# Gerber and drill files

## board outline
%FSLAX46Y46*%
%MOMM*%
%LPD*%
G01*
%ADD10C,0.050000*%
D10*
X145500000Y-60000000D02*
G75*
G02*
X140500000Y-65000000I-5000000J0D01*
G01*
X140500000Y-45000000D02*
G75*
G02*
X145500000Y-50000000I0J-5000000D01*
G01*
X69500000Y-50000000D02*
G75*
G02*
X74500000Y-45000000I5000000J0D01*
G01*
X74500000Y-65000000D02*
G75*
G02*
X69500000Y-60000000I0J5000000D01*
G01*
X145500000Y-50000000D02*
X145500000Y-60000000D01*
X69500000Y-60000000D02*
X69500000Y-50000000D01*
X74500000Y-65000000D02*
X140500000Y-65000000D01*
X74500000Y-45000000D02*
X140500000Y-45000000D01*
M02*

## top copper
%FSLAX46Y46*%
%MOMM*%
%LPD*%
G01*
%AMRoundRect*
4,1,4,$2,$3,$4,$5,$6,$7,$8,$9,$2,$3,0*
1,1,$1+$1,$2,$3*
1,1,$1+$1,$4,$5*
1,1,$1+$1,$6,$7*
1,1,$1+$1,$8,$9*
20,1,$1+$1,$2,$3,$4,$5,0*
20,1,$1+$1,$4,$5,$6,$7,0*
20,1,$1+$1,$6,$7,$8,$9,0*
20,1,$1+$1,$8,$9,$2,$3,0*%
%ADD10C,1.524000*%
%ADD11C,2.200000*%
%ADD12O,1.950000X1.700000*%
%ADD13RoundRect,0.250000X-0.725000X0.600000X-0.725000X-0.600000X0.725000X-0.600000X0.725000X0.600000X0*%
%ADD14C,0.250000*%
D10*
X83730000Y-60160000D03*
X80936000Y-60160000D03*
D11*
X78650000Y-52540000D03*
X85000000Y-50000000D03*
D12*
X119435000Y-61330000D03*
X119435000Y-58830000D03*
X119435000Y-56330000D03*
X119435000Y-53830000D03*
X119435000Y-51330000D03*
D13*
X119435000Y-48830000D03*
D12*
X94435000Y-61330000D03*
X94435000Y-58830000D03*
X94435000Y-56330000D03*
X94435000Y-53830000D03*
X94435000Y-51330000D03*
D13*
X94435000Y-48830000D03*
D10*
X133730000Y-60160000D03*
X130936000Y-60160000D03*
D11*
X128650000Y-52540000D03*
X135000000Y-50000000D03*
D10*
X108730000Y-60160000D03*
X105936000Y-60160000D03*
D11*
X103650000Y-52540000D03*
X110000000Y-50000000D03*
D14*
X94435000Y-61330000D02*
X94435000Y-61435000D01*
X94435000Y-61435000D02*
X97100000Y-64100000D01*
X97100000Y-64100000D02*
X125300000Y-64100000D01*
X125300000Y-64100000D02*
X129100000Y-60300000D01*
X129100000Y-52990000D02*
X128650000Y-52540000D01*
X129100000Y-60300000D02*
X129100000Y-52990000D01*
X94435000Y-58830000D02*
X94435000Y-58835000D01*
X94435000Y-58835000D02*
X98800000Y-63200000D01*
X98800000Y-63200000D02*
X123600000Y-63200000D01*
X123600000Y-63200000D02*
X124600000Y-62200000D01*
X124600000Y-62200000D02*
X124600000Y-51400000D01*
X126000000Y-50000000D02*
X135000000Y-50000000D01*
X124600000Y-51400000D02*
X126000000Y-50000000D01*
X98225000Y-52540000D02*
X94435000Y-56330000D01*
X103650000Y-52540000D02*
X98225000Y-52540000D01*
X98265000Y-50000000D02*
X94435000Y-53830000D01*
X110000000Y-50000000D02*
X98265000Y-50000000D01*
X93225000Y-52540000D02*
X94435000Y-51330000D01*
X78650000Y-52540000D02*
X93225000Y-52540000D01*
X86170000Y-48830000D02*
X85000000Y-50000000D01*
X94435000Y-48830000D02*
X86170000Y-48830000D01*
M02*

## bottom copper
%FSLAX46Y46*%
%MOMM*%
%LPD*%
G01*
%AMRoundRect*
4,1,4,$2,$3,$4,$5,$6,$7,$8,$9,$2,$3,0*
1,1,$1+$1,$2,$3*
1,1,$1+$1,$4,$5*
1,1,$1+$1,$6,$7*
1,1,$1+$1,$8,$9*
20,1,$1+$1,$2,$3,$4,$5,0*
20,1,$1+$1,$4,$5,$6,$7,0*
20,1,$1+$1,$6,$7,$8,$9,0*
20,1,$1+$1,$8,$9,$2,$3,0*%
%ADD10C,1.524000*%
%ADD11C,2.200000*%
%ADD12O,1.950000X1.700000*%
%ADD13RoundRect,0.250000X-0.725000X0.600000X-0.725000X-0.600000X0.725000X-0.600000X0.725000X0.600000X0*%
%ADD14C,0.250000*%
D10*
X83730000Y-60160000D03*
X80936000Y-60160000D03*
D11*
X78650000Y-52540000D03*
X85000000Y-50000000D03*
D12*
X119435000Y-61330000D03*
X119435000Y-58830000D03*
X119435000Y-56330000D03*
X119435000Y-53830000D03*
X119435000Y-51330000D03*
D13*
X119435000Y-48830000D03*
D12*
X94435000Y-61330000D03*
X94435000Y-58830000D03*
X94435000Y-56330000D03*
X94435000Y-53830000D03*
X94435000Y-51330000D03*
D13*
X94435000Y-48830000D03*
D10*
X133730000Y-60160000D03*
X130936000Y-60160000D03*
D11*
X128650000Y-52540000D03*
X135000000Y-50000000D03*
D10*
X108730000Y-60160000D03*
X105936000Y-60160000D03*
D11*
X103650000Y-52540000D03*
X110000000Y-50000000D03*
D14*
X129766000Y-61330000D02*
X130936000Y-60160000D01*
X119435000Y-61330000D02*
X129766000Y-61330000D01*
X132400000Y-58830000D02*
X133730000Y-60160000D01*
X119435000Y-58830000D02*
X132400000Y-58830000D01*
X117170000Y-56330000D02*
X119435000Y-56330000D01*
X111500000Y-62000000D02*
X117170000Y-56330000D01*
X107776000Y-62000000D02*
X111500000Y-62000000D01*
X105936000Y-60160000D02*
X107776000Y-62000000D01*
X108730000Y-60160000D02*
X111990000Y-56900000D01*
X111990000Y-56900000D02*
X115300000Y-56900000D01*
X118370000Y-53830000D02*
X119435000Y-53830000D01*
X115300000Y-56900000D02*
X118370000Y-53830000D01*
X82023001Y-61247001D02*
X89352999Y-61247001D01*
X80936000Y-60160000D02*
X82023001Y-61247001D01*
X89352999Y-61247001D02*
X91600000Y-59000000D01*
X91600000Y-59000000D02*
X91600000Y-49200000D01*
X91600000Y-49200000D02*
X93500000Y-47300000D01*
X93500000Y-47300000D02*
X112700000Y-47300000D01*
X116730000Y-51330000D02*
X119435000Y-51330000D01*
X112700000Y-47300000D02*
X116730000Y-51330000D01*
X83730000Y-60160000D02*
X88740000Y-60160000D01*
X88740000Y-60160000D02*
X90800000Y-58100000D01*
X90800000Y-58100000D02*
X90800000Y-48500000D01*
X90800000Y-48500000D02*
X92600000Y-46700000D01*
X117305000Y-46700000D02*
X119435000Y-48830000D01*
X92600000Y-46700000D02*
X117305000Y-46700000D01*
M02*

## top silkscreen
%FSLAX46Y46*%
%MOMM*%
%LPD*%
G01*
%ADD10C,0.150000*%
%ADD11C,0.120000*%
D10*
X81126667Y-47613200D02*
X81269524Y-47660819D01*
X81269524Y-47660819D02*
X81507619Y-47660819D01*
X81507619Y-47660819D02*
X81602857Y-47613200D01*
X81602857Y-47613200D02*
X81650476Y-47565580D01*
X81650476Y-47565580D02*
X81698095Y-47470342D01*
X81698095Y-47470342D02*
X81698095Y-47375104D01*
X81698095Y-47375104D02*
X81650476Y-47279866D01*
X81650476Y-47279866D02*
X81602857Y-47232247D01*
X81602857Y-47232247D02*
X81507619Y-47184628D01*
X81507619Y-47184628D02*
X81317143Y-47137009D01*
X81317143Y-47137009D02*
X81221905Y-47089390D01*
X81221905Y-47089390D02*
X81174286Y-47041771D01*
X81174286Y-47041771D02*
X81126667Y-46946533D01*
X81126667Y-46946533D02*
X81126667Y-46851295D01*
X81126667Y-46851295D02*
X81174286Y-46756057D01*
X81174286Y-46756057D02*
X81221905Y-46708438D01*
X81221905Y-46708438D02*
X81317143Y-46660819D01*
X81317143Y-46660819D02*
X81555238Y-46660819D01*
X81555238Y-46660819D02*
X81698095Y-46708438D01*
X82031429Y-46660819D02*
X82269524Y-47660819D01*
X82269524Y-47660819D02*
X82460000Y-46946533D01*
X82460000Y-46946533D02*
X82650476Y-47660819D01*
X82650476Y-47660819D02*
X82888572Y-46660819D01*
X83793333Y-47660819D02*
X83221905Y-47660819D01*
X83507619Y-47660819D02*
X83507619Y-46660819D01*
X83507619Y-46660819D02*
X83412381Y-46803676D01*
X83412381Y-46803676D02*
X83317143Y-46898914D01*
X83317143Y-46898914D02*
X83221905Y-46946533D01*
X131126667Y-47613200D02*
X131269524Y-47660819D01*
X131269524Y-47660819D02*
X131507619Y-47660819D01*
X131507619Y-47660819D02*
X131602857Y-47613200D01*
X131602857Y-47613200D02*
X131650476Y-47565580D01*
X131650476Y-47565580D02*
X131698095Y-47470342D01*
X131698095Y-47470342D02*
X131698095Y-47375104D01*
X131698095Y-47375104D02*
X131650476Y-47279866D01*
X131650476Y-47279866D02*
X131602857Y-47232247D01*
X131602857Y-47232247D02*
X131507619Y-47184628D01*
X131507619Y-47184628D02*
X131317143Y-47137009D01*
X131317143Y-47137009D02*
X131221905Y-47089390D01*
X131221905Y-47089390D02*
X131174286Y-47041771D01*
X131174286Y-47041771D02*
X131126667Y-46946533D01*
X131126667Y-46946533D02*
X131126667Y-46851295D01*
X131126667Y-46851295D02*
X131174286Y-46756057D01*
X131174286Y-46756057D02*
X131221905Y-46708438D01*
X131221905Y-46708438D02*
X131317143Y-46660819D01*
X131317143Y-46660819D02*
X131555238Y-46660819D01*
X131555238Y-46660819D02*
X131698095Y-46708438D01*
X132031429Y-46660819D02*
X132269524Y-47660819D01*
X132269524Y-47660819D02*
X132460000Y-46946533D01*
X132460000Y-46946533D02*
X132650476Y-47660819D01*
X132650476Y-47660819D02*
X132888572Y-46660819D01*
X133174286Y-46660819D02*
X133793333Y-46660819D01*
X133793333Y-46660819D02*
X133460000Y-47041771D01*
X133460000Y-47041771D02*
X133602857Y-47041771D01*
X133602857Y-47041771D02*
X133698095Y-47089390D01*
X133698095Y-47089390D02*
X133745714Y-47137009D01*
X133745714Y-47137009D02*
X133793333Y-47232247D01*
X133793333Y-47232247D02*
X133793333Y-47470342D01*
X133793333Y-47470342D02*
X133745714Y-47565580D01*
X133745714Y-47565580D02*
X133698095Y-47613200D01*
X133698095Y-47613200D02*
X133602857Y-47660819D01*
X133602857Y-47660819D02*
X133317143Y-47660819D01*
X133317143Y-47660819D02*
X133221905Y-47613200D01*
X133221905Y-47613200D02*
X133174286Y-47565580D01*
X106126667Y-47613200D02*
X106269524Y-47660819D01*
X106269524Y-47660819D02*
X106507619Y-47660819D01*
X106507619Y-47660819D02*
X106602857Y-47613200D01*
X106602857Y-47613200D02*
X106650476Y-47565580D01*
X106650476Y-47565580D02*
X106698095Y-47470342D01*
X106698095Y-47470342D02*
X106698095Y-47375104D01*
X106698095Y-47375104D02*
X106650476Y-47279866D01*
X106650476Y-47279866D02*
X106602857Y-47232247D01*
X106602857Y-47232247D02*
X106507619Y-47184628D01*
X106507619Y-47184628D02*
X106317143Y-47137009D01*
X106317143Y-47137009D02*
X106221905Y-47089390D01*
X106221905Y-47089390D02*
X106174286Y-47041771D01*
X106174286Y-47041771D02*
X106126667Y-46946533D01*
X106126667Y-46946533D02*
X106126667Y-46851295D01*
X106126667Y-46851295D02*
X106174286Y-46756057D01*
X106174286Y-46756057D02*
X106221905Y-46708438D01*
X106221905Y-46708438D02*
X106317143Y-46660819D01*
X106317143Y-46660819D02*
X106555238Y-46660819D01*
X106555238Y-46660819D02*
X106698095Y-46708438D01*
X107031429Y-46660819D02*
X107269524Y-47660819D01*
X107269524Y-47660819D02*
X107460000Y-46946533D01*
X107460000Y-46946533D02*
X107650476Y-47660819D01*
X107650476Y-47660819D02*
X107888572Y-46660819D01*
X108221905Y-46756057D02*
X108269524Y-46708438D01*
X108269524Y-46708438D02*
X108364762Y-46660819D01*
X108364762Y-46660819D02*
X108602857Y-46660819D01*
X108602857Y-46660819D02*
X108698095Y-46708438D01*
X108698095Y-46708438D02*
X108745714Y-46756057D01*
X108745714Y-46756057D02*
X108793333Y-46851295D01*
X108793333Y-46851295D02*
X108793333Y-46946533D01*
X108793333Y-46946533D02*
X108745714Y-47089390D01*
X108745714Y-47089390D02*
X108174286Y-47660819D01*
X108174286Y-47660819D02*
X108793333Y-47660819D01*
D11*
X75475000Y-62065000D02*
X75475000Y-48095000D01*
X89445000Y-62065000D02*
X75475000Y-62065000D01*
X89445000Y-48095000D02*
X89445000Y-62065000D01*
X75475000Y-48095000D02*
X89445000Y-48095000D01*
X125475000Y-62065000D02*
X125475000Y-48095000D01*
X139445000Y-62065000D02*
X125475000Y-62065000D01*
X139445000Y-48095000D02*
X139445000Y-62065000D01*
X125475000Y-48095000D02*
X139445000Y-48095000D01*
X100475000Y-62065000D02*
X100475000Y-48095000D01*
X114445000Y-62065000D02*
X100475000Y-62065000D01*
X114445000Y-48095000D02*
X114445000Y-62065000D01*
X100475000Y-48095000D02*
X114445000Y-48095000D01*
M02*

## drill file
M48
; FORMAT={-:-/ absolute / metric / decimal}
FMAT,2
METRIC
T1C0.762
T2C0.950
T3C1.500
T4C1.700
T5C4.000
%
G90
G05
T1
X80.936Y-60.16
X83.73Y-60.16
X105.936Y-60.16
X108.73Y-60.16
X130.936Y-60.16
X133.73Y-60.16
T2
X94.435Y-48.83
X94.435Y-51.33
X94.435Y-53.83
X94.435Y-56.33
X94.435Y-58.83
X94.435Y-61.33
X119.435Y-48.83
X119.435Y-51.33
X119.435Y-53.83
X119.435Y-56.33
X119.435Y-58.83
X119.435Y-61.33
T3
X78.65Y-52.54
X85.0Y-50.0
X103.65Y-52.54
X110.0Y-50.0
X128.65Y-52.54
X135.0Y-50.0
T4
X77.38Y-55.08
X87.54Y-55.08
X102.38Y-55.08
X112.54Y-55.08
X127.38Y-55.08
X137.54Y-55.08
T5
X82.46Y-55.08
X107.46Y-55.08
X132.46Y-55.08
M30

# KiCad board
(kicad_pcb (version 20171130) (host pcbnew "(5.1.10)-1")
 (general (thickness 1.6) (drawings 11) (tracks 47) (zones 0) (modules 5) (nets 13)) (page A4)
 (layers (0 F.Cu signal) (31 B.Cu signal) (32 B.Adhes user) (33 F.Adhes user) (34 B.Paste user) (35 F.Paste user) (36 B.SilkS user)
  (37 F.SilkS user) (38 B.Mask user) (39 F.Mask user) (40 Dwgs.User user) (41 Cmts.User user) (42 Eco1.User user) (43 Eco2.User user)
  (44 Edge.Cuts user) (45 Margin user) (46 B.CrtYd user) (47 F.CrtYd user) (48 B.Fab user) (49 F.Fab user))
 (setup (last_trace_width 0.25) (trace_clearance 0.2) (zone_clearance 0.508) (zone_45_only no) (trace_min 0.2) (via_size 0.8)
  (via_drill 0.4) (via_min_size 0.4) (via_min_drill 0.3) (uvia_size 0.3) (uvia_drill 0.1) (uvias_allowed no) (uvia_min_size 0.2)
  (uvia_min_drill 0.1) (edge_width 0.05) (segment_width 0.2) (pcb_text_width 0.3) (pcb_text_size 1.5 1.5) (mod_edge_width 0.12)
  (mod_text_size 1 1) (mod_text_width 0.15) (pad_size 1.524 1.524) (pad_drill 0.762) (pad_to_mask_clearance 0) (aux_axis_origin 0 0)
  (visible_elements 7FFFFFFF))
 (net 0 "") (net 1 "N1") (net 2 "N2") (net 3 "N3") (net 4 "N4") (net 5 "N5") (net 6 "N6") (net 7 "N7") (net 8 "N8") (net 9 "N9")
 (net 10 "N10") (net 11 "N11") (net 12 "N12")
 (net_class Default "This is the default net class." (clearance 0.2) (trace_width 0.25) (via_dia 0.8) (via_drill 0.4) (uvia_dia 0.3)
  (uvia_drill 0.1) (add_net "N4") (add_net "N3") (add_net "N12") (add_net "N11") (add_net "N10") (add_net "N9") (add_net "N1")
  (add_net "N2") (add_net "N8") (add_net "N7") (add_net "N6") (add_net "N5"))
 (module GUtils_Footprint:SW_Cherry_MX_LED (layer F.Cu) (at 85 50)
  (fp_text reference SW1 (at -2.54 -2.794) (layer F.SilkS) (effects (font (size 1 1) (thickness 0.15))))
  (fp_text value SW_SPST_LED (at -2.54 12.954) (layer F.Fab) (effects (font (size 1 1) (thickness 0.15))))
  (fp_line (start -9.525 12.065) (end -9.525 -1.905) (layer F.SilkS) (width 0.12))
  (fp_line (start 4.445 12.065) (end -9.525 12.065) (layer F.SilkS) (width 0.12))
  (fp_line (start 4.445 -1.905) (end 4.445 12.065) (layer F.SilkS) (width 0.12))
  (fp_line (start -9.525 -1.905) (end 4.445 -1.905) (layer F.SilkS) (width 0.12))
  (pad 4 thru_hole circle (at -1.27 10.16) (size 1.524 1.524) (drill 0.762) (layers *.Cu *.Mask) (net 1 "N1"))
  (pad 3 thru_hole circle (at -4.064 10.16) (size 1.524 1.524) (drill 0.762) (layers *.Cu *.Mask) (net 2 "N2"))
  (pad "" np_thru_hole circle (at 2.54 5.08) (size 1.7 1.7) (drill 1.7) (layers *.Cu *.Mask))
  (pad "" np_thru_hole circle (at -7.62 5.08) (size 1.7 1.7) (drill 1.7) (layers *.Cu *.Mask))
  (pad "" np_thru_hole circle (at -2.54 5.08) (size 4 4) (drill 4) (layers *.Cu *.Mask))
  (pad 2 thru_hole circle (at -6.35 2.54) (size 2.2 2.2) (drill 1.5) (layers *.Cu *.Mask) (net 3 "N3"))
  (pad 1 thru_hole circle (at 0 0) (size 2.2 2.2) (drill 1.5) (layers *.Cu *.Mask) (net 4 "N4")))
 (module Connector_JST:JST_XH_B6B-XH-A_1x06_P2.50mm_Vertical (layer B.Cu) (at 119.435 48.83 270)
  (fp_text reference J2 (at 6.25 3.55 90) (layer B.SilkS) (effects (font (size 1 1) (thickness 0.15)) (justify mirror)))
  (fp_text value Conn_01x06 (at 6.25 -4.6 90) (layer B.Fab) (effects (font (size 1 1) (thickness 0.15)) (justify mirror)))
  (pad 6 thru_hole oval (at 12.5 0 270) (size 1.7 1.95) (drill 0.95) (layers *.Cu *.Mask) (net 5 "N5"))
  (pad 5 thru_hole oval (at 10 0 270) (size 1.7 1.95) (drill 0.95) (layers *.Cu *.Mask) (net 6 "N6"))
  (pad 4 thru_hole oval (at 7.5 0 270) (size 1.7 1.95) (drill 0.95) (layers *.Cu *.Mask) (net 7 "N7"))
  (pad 3 thru_hole oval (at 5 0 270) (size 1.7 1.95) (drill 0.95) (layers *.Cu *.Mask) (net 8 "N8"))
  (pad 2 thru_hole oval (at 2.5 0 270) (size 1.7 1.95) (drill 0.95) (layers *.Cu *.Mask) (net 2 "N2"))
  (pad 1 thru_hole roundrect (at 0 0 270) (size 1.7 1.95) (drill 0.95) (layers *.Cu *.Mask) (roundrect_rratio 0.147059) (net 1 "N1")))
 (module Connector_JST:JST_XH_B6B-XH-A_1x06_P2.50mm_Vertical (layer B.Cu) (at 94.435 48.83 270)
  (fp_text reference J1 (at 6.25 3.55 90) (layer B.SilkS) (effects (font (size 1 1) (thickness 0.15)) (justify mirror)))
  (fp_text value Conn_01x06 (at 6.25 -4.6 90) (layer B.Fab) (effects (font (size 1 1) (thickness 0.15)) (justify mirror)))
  (pad 6 thru_hole oval (at 12.5 0 270) (size 1.7 1.95) (drill 0.95) (layers *.Cu *.Mask) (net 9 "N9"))
  (pad 5 thru_hole oval (at 10 0 270) (size 1.7 1.95) (drill 0.95) (layers *.Cu *.Mask) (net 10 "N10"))
  (pad 4 thru_hole oval (at 7.5 0 270) (size 1.7 1.95) (drill 0.95) (layers *.Cu *.Mask) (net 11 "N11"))
  (pad 3 thru_hole oval (at 5 0 270) (size 1.7 1.95) (drill 0.95) (layers *.Cu *.Mask) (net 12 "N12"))
  (pad 2 thru_hole oval (at 2.5 0 270) (size 1.7 1.95) (drill 0.95) (layers *.Cu *.Mask) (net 3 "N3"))
  (pad 1 thru_hole roundrect (at 0 0 270) (size 1.7 1.95) (drill 0.95) (layers *.Cu *.Mask) (roundrect_rratio 0.147059) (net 4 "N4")))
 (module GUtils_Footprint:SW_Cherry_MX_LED (layer F.Cu) (at 135 50)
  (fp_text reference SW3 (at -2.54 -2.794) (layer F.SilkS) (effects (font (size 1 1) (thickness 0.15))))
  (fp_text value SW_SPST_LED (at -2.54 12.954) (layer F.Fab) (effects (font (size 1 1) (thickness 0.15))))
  (fp_line (start -9.525 12.065) (end -9.525 -1.905) (layer F.SilkS) (width 0.12))
  (fp_line (start 4.445 12.065) (end -9.525 12.065) (layer F.SilkS) (width 0.12))
  (fp_line (start 4.445 -1.905) (end 4.445 12.065) (layer F.SilkS) (width 0.12))
  (fp_line (start -9.525 -1.905) (end 4.445 -1.905) (layer F.SilkS) (width 0.12))
  (pad 4 thru_hole circle (at -1.27 10.16) (size 1.524 1.524) (drill 0.762) (layers *.Cu *.Mask) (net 6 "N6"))
  (pad 3 thru_hole circle (at -4.064 10.16) (size 1.524 1.524) (drill 0.762) (layers *.Cu *.Mask) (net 5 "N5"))
  (pad "" np_thru_hole circle (at 2.54 5.08) (size 1.7 1.7) (drill 1.7) (layers *.Cu *.Mask))
  (pad "" np_thru_hole circle (at -7.62 5.08) (size 1.7 1.7) (drill 1.7) (layers *.Cu *.Mask))
  (pad "" np_thru_hole circle (at -2.54 5.08) (size 4 4) (drill 4) (layers *.Cu *.Mask))
  (pad 2 thru_hole circle (at -6.35 2.54) (size 2.2 2.2) (drill 1.5) (layers *.Cu *.Mask) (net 9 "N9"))
  (pad 1 thru_hole circle (at 0 0) (size 2.2 2.2) (drill 1.5) (layers *.Cu *.Mask) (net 10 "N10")))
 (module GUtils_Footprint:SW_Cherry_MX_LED (layer F.Cu) (at 110 50)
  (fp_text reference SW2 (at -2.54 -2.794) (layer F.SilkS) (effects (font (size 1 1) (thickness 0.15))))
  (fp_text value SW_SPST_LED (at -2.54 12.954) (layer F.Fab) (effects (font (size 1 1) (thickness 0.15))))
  (fp_line (start -9.525 12.065) (end -9.525 -1.905) (layer F.SilkS) (width 0.12))
  (fp_line (start 4.445 12.065) (end -9.525 12.065) (layer F.SilkS) (width 0.12))
  (fp_line (start 4.445 -1.905) (end 4.445 12.065) (layer F.SilkS) (width 0.12))
  (fp_line (start -9.525 -1.905) (end 4.445 -1.905) (layer F.SilkS) (width 0.12))
  (pad 4 thru_hole circle (at -1.27 10.16) (size 1.524 1.524) (drill 0.762) (layers *.Cu *.Mask) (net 8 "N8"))
  (pad 3 thru_hole circle (at -4.064 10.16) (size 1.524 1.524) (drill 0.762) (layers *.Cu *.Mask) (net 7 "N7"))
  (pad "" np_thru_hole circle (at 2.54 5.08) (size 1.7 1.7) (drill 1.7) (layers *.Cu *.Mask))
  (pad "" np_thru_hole circle (at -7.62 5.08) (size 1.7 1.7) (drill 1.7) (layers *.Cu *.Mask))
  (pad "" np_thru_hole circle (at -2.54 5.08) (size 4 4) (drill 4) (layers *.Cu *.Mask))
  (pad 2 thru_hole circle (at -6.35 2.54) (size 2.2 2.2) (drill 1.5) (layers *.Cu *.Mask) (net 11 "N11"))
  (pad 1 thru_hole circle (at 0 0) (size 2.2 2.2) (drill 1.5) (layers *.Cu *.Mask) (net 12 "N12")))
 (gr_arc (start 140.5 60) (end 140.5 65) (angle -90) (layer Edge.Cuts) (width 0.05))
 (gr_arc (start 140.5 50) (end 145.5 50) (angle -90) (layer Edge.Cuts) (width 0.05))
 (gr_arc (start 74.5 50) (end 74.5 45) (angle -90) (layer Edge.Cuts) (width 0.05))
 (gr_arc (start 74.5 60) (end 69.5 60) (angle -90) (layer Edge.Cuts) (width 0.05))
 (gr_line (start 145.5 50) (end 145.5 60) (layer Edge.Cuts) (width 0.05))
 (gr_line (start 69.5 60) (end 69.5 50) (layer Edge.Cuts) (width 0.05))
 (gr_line (start 74.5 65) (end 140.5 65) (layer Edge.Cuts) (width 0.05))
 (gr_line (start 74.5 45) (end 140.5 45) (layer Edge.Cuts) (width 0.05))
 (segment (start 94.435 61.33) (end 94.435 61.435) (width 0.25) (layer F.Cu) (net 9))
 (segment (start 94.435 61.435) (end 97.1 64.1) (width 0.25) (layer F.Cu) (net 9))
 (segment (start 97.1 64.1) (end 125.3 64.1) (width 0.25) (layer F.Cu) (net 9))
 (segment (start 125.3 64.1) (end 129.1 60.3) (width 0.25) (layer F.Cu) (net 9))
 (segment (start 129.1 52.99) (end 128.65 52.54) (width 0.25) (layer F.Cu) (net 9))
 (segment (start 129.1 60.3) (end 129.1 52.99) (width 0.25) (layer F.Cu) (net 9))
 (segment (start 94.435 58.83) (end 94.435 58.835) (width 0.25) (layer F.Cu) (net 10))
 (segment (start 94.435 58.835) (end 98.8 63.2) (width 0.25) (layer F.Cu) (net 10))
 (segment (start 98.8 63.2) (end 123.6 63.2) (width 0.25) (layer F.Cu) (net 10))
 (segment (start 123.6 63.2) (end 124.6 62.2) (width 0.25) (layer F.Cu) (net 10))
 (segment (start 124.6 62.2) (end 124.6 51.4) (width 0.25) (layer F.Cu) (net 10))
 (segment (start 126 50) (end 135 50) (width 0.25) (layer F.Cu) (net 10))
 (segment (start 124.6 51.4) (end 126 50) (width 0.25) (layer F.Cu) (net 10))
 (segment (start 98.225 52.54) (end 94.435 56.33) (width 0.25) (layer F.Cu) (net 11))
 (segment (start 103.65 52.54) (end 98.225 52.54) (width 0.25) (layer F.Cu) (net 11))
 (segment (start 98.265 50) (end 94.435 53.83) (width 0.25) (layer F.Cu) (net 12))
 (segment (start 110 50) (end 98.265 50) (width 0.25) (layer F.Cu) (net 12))
 (segment (start 93.225 52.54) (end 94.435 51.33) (width 0.25) (layer F.Cu) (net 3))
 (segment (start 78.65 52.54) (end 93.225 52.54) (width 0.25) (layer F.Cu) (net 3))
 (segment (start 86.17 48.83) (end 85 50) (width 0.25) (layer F.Cu) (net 4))
 (segment (start 94.435 48.83) (end 86.17 48.83) (width 0.25) (layer F.Cu) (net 4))
 (segment (start 129.766 61.33) (end 130.936 60.16) (width 0.25) (layer B.Cu) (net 5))
 (segment (start 119.435 61.33) (end 129.766 61.33) (width 0.25) (layer B.Cu) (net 5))
 (segment (start 132.4 58.83) (end 133.73 60.16) (width 0.25) (layer B.Cu) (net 6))
 (segment (start 119.435 58.83) (end 132.4 58.83) (width 0.25) (layer B.Cu) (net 6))
 (segment (start 117.17 56.33) (end 119.435 56.33) (width 0.25) (layer B.Cu) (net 7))
 (segment (start 111.5 62) (end 117.17 56.33) (width 0.25) (layer B.Cu) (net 7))
 (segment (start 107.776 62) (end 111.5 62) (width 0.25) (layer B.Cu) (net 7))
 (segment (start 105.936 60.16) (end 107.776 62) (width 0.25) (layer B.Cu) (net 7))
 (segment (start 108.73 60.16) (end 111.99 56.9) (width 0.25) (layer B.Cu) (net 8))
 (segment (start 111.99 56.9) (end 115.3 56.9) (width 0.25) (layer B.Cu) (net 8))
 (segment (start 118.37 53.83) (end 119.435 53.83) (width 0.25) (layer B.Cu) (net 8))
 (segment (start 115.3 56.9) (end 118.37 53.83) (width 0.25) (layer B.Cu) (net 8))
 (segment (start 82.023001 61.247001) (end 89.352999 61.247001) (width 0.25) (layer B.Cu) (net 2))
 (segment (start 80.936 60.16) (end 82.023001 61.247001) (width 0.25) (layer B.Cu) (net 2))
 (segment (start 89.352999 61.247001) (end 91.6 59) (width 0.25) (layer B.Cu) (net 2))
 (segment (start 91.6 59) (end 91.6 49.2) (width 0.25) (layer B.Cu) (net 2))
 (segment (start 91.6 49.2) (end 93.5 47.3) (width 0.25) (layer B.Cu) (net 2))
 (segment (start 93.5 47.3) (end 112.7 47.3) (width 0.25) (layer B.Cu) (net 2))
 (segment (start 116.73 51.33) (end 119.435 51.33) (width 0.25) (layer B.Cu) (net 2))
 (segment (start 112.7 47.3) (end 116.73 51.33) (width 0.25) (layer B.Cu) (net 2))
 (segment (start 83.73 60.16) (end 88.74 60.16) (width 0.25) (layer B.Cu) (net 1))
 (segment (start 88.74 60.16) (end 90.8 58.1) (width 0.25) (layer B.Cu) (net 1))
 (segment (start 90.8 58.1) (end 90.8 48.5) (width 0.25) (layer B.Cu) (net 1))
 (segment (start 90.8 48.5) (end 92.6 46.7) (width 0.25) (layer B.Cu) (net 1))
 (segment (start 117.305 46.7) (end 119.435 48.83) (width 0.25) (layer B.Cu) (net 1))
 (segment (start 92.6 46.7) (end 117.305 46.7) (width 0.25) (layer B.Cu) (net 1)))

